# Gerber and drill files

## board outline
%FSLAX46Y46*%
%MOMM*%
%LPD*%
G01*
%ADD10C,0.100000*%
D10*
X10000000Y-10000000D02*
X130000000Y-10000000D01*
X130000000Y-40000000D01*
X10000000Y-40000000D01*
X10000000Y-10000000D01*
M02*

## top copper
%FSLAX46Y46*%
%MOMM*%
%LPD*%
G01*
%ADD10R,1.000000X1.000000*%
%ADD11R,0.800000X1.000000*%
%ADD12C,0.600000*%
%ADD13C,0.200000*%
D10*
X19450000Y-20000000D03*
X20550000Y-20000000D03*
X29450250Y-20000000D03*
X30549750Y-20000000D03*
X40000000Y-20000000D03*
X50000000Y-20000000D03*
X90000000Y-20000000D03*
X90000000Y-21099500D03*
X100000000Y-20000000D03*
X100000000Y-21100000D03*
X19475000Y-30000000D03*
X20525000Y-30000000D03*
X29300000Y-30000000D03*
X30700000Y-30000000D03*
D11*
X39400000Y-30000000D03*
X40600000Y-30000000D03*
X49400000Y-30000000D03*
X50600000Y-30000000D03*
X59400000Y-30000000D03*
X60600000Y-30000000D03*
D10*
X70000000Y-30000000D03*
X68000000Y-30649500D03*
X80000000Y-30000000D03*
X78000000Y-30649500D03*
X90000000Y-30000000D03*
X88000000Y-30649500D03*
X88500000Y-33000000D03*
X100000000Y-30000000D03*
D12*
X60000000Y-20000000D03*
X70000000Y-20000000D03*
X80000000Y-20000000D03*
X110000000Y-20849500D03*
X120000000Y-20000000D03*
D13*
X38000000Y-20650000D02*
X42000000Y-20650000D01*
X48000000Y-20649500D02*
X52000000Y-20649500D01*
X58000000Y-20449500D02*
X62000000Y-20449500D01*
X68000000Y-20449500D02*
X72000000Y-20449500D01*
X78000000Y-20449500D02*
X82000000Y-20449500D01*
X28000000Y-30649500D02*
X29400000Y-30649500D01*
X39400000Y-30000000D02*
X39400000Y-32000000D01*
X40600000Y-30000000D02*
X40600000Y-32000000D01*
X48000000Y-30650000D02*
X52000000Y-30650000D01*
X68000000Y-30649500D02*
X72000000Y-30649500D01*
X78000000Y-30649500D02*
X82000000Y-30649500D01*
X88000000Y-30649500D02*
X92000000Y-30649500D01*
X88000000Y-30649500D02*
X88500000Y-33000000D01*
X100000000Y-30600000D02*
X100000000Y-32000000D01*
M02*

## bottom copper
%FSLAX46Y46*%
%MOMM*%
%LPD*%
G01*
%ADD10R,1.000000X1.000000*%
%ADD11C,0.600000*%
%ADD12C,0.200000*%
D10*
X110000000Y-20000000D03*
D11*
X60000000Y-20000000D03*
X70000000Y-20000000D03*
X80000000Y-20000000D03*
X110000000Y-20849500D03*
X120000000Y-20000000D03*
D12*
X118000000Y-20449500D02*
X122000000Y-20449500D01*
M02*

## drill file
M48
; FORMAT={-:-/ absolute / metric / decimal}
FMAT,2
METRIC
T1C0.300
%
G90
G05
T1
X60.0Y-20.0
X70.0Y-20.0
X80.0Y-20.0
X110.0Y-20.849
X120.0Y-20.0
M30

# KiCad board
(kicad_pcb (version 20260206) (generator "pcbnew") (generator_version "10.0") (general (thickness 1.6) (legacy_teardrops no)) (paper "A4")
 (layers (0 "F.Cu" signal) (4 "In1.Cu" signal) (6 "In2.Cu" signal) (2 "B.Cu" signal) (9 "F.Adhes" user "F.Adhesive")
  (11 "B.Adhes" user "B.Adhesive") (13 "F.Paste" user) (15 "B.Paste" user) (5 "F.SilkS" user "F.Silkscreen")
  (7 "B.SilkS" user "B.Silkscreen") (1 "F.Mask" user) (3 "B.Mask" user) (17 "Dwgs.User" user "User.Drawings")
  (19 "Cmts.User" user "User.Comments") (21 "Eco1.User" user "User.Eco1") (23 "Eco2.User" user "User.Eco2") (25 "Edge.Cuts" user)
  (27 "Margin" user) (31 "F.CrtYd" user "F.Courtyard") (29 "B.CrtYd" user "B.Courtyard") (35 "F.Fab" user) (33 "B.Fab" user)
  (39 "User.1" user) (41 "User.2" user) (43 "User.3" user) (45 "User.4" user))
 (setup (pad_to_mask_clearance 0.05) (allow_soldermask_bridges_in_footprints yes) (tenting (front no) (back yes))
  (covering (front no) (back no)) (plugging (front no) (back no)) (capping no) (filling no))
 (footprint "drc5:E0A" (layer "F.Cu") (at 19.45 20)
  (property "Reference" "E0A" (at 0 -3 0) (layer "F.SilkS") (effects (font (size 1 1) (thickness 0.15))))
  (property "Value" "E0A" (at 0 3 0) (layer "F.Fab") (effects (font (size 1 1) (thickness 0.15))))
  (pad "1" smd rect (at 0 0) (size 1 1) (layers "F.Cu" "F.Mask" "F.Paste") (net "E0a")))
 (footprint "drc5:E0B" (layer "F.Cu") (at 20.55 20)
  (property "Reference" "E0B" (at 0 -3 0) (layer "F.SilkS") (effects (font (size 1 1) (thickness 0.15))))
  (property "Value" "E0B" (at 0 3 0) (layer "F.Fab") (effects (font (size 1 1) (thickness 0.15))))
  (pad "1" smd rect (at 0 0) (size 1 1) (layers "F.Cu" "F.Mask" "F.Paste") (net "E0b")))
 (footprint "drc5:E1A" (layer "F.Cu") (at 29.45025 20)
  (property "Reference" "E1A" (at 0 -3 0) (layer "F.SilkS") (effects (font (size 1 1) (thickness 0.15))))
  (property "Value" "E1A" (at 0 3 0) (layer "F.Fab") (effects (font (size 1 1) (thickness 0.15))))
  (pad "1" smd rect (at 0 0) (size 1 1) (layers "F.Cu" "F.Mask" "F.Paste") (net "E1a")))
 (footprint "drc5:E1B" (layer "F.Cu") (at 30.54975 20)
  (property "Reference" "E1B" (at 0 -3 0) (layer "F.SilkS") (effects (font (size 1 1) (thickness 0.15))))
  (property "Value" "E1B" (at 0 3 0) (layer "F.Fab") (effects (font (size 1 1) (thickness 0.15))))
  (pad "1" smd rect (at 0 0) (size 1 1) (layers "F.Cu" "F.Mask" "F.Paste") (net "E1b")))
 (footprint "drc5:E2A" (layer "F.Cu") (at 40 20)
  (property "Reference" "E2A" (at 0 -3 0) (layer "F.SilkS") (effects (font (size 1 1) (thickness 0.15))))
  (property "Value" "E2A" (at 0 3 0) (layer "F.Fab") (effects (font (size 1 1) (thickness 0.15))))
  (pad "1" smd rect (at 0 0) (size 1 1) (layers "F.Cu" "F.Mask" "F.Paste") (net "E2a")))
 (segment (start 38 20.65) (end 42 20.65) (width 0.2) (layer "F.Cu") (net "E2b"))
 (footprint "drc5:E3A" (layer "F.Cu") (at 50 20)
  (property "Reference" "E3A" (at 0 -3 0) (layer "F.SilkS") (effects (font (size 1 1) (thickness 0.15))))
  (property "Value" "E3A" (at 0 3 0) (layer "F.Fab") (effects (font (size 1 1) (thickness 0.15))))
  (pad "1" smd rect (at 0 0) (size 1 1) (layers "F.Cu" "F.Mask" "F.Paste") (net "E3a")))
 (segment (start 48 20.6495) (end 52 20.6495) (width 0.2) (layer "F.Cu") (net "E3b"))
 (via (at 60 20) (size 0.6) (drill 0.3) (layers "F.Cu" "B.Cu") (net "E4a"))
 (segment (start 58 20.4495) (end 62 20.4495) (width 0.2) (layer "F.Cu") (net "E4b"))
 (via (at 70 20) (size 0.6) (drill 0.3) (layers "F.Cu" "B.Cu") (tenting (front yes) (back yes)) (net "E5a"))
 (segment (start 68 20.4495) (end 72 20.4495) (width 0.2) (layer "F.Cu") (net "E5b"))
 (via (at 80 20) (size 0.6) (drill 0.3) (layers "F.Cu" "B.Cu") (tenting (front none) (back none)) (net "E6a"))
 (segment (start 78 20.4495) (end 82 20.4495) (width 0.2) (layer "F.Cu") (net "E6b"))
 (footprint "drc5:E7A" (layer "F.Cu") (at 90 20)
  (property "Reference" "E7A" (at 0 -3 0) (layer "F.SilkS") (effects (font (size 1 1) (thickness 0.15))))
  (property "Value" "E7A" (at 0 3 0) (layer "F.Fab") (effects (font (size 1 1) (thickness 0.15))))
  (pad "1" smd rect (at 0 0) (size 1 1) (layers "F.Cu" "F.Mask" "F.Paste") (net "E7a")))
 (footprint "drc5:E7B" (layer "F.Cu") (at 90 21.0995)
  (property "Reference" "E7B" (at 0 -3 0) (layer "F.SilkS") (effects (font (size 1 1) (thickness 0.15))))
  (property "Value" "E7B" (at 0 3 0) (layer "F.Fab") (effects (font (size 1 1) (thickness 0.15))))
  (pad "1" smd rect (at 0 0) (size 1 1) (layers "F.Cu") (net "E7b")))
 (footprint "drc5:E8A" (layer "F.Cu") (at 100 20)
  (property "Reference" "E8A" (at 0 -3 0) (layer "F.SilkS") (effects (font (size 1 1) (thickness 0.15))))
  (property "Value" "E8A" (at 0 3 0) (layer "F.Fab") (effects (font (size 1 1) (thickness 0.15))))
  (pad "1" smd rect (at 0 0) (size 1 1) (layers "F.Cu" "F.Mask" "F.Paste") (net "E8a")))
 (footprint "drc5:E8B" (layer "F.Cu") (at 100 21.1)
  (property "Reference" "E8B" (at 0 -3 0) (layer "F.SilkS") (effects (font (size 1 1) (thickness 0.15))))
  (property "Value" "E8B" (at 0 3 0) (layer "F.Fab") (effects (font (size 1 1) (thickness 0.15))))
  (pad "1" smd rect (at 0 0) (size 1 1) (layers "F.Cu") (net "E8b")))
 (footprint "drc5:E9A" (layer "B.Cu") (at 110 20)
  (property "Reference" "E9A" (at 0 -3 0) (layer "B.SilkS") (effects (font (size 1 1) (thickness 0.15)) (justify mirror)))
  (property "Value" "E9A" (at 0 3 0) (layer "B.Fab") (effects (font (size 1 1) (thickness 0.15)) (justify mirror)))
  (pad "1" smd rect (at 0 0) (size 1 1) (layers "B.Cu" "B.Mask" "B.Paste") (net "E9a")))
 (via (at 110 20.8495) (size 0.6) (drill 0.3) (layers "F.Cu" "B.Cu") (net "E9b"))
 (via (at 120 20) (size 0.6) (drill 0.3) (layers "F.Cu" "B.Cu") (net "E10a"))
 (segment (start 118 20.4495) (end 122 20.4495) (width 0.2) (layer "B.Cu") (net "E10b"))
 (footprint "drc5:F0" (layer "F.Cu") (at 20 30)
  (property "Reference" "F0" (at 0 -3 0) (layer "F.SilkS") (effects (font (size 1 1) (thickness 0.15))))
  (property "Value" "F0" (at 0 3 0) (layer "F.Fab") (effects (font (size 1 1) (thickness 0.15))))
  (pad "1" smd rect (at -0.525 0) (size 1 1) (layers "F.Cu" "F.Mask" "F.Paste") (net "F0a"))
  (pad "2" smd rect (at 0.525 0) (size 1 1) (layers "F.Cu" "F.Mask" "F.Paste") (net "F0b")))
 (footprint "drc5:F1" (layer "F.Cu") (at 30 30)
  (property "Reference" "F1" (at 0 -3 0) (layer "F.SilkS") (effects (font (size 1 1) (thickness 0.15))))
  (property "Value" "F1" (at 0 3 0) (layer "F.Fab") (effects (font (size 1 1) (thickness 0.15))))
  (pad "1" smd rect (at -0.7 0) (size 1 1) (layers "F.Cu" "F.Mask" "F.Paste") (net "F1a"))
  (pad "2" smd rect (at 0.7 0) (size 1 1) (layers "F.Cu" "F.Mask" "F.Paste") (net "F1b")))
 (segment (start 28 30.6495) (end 29.4 30.6495) (width 0.2) (layer "F.Cu") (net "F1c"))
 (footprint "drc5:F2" (layer "F.Cu") (at 40 30)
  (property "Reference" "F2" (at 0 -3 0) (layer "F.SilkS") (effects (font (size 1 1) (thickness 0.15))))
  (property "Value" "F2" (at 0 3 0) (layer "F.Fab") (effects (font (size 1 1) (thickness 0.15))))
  (pad "1" smd rect (at -0.6 0) (size 0.8 1) (layers "F.Cu" "F.Mask" "F.Paste") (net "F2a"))
  (pad "2" smd rect (at 0.6 0) (size 0.8 1) (layers "F.Cu" "F.Mask" "F.Paste") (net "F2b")))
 (segment (start 39.4 30) (end 39.4 32) (width 0.2) (layer "F.Cu") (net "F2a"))
 (segment (start 40.6 30) (end 40.6 32) (width 0.2) (layer "F.Cu") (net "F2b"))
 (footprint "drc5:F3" (layer "F.Cu") (at 50 30)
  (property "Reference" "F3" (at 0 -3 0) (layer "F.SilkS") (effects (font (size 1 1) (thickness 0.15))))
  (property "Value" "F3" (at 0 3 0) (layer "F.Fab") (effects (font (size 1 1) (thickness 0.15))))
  (pad "1" smd rect (at -0.6 0) (size 0.8 1) (layers "F.Cu" "F.Mask" "F.Paste") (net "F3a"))
  (pad "2" smd rect (at 0.6 0) (size 0.8 1) (layers "F.Cu" "F.Mask" "F.Paste") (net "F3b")))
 (segment (start 48 30.65) (end 52 30.65) (width 0.2) (layer "F.Cu") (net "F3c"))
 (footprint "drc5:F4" (layer "F.Cu") (at 60 30)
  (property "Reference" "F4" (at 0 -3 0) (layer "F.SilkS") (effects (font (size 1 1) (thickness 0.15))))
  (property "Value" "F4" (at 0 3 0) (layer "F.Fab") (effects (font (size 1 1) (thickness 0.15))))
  (pad "1" smd rect (at -0.6 0) (size 0.8 1) (layers "F.Cu" "F.Mask" "F.Paste") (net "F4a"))
  (pad "2" smd rect (at 0.6 0) (size 0.8 1) (layers "F.Cu" "F.Mask" "F.Paste") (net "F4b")))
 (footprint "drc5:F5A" (layer "F.Cu") (at 70 30)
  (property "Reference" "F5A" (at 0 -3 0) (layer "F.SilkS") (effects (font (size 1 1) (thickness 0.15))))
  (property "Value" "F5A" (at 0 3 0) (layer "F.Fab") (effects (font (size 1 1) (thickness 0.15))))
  (pad "1" smd rect (at 0 0) (size 1 1) (layers "F.Cu" "F.Mask" "F.Paste") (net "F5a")))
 (segment (start 68 30.6495) (end 72 30.6495) (width 0.2) (layer "F.Cu") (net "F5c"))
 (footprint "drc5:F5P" (layer "F.Cu") (at 68 30.6495)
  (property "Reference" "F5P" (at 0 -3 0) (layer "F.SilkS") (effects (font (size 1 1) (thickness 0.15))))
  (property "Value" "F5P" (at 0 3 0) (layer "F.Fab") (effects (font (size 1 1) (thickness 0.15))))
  (pad "1" smd rect (at 0 0) (size 1 1) (layers "F.Cu" "F.Mask" "F.Paste") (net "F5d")))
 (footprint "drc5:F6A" (layer "F.Cu") (at 80 30)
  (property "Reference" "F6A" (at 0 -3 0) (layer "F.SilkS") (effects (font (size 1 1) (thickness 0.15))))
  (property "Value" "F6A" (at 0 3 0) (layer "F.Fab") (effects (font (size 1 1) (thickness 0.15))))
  (pad "1" smd rect (at 0 0) (size 1 1) (layers "F.Cu" "F.Mask" "F.Paste") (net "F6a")))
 (segment (start 78 30.6495) (end 82 30.6495) (width 0.2) (layer "F.Cu") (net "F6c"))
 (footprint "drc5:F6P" (layer "F.Cu") (at 78 30.6495)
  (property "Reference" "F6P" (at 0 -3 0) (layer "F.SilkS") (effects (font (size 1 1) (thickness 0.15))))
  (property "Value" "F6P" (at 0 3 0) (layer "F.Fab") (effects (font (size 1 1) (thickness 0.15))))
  (pad "1" smd rect (at 0 0) (size 1 1) (layers "F.Cu" "F.Mask" "F.Paste") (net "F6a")))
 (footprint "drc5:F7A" (layer "F.Cu") (at 90 30)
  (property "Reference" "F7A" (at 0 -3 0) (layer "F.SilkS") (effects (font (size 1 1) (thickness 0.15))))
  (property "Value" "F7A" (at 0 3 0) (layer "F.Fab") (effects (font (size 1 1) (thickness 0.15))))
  (pad "1" smd rect (at 0 0) (size 1 1) (layers "F.Cu" "F.Mask" "F.Paste") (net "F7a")))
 (segment (start 88 30.6495) (end 92 30.6495) (width 0.2) (layer "F.Cu") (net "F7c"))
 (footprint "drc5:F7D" (layer "F.Cu") (at 88 30.6495)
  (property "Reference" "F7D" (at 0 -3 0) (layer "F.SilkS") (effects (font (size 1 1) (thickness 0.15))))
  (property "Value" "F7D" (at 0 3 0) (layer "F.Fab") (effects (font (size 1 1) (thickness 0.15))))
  (pad "1" smd rect (at 0 0) (size 1 1) (layers "F.Cu" "F.Mask" "F.Paste") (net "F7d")))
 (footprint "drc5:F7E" (layer "F.Cu") (at 88.5 33)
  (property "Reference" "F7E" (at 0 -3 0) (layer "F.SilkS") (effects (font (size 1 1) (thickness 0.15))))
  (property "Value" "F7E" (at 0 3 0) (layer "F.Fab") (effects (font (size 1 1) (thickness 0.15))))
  (pad "1" smd rect (at 0 0) (size 1 1) (layers "F.Cu" "F.Mask" "F.Paste") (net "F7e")))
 (segment (start 88 30.6495) (end 88.5 33) (width 0.2) (layer "F.Cu") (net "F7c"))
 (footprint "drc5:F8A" (layer "F.Cu") (at 100 30)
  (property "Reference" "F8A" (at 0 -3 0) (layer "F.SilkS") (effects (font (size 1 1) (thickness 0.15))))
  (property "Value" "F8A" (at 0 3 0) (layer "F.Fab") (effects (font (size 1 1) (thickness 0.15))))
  (pad "1" smd rect (at 0 0) (size 1 1) (layers "F.Cu" "F.Mask" "F.Paste") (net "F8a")))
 (segment (start 100 30.6) (end 100 32) (width 0.2) (layer "F.Cu") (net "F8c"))
 (gr_rect (start 10 10) (end 130 40) (stroke (width 0.1) (type solid)) (fill no) (layer "Edge.Cuts")))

